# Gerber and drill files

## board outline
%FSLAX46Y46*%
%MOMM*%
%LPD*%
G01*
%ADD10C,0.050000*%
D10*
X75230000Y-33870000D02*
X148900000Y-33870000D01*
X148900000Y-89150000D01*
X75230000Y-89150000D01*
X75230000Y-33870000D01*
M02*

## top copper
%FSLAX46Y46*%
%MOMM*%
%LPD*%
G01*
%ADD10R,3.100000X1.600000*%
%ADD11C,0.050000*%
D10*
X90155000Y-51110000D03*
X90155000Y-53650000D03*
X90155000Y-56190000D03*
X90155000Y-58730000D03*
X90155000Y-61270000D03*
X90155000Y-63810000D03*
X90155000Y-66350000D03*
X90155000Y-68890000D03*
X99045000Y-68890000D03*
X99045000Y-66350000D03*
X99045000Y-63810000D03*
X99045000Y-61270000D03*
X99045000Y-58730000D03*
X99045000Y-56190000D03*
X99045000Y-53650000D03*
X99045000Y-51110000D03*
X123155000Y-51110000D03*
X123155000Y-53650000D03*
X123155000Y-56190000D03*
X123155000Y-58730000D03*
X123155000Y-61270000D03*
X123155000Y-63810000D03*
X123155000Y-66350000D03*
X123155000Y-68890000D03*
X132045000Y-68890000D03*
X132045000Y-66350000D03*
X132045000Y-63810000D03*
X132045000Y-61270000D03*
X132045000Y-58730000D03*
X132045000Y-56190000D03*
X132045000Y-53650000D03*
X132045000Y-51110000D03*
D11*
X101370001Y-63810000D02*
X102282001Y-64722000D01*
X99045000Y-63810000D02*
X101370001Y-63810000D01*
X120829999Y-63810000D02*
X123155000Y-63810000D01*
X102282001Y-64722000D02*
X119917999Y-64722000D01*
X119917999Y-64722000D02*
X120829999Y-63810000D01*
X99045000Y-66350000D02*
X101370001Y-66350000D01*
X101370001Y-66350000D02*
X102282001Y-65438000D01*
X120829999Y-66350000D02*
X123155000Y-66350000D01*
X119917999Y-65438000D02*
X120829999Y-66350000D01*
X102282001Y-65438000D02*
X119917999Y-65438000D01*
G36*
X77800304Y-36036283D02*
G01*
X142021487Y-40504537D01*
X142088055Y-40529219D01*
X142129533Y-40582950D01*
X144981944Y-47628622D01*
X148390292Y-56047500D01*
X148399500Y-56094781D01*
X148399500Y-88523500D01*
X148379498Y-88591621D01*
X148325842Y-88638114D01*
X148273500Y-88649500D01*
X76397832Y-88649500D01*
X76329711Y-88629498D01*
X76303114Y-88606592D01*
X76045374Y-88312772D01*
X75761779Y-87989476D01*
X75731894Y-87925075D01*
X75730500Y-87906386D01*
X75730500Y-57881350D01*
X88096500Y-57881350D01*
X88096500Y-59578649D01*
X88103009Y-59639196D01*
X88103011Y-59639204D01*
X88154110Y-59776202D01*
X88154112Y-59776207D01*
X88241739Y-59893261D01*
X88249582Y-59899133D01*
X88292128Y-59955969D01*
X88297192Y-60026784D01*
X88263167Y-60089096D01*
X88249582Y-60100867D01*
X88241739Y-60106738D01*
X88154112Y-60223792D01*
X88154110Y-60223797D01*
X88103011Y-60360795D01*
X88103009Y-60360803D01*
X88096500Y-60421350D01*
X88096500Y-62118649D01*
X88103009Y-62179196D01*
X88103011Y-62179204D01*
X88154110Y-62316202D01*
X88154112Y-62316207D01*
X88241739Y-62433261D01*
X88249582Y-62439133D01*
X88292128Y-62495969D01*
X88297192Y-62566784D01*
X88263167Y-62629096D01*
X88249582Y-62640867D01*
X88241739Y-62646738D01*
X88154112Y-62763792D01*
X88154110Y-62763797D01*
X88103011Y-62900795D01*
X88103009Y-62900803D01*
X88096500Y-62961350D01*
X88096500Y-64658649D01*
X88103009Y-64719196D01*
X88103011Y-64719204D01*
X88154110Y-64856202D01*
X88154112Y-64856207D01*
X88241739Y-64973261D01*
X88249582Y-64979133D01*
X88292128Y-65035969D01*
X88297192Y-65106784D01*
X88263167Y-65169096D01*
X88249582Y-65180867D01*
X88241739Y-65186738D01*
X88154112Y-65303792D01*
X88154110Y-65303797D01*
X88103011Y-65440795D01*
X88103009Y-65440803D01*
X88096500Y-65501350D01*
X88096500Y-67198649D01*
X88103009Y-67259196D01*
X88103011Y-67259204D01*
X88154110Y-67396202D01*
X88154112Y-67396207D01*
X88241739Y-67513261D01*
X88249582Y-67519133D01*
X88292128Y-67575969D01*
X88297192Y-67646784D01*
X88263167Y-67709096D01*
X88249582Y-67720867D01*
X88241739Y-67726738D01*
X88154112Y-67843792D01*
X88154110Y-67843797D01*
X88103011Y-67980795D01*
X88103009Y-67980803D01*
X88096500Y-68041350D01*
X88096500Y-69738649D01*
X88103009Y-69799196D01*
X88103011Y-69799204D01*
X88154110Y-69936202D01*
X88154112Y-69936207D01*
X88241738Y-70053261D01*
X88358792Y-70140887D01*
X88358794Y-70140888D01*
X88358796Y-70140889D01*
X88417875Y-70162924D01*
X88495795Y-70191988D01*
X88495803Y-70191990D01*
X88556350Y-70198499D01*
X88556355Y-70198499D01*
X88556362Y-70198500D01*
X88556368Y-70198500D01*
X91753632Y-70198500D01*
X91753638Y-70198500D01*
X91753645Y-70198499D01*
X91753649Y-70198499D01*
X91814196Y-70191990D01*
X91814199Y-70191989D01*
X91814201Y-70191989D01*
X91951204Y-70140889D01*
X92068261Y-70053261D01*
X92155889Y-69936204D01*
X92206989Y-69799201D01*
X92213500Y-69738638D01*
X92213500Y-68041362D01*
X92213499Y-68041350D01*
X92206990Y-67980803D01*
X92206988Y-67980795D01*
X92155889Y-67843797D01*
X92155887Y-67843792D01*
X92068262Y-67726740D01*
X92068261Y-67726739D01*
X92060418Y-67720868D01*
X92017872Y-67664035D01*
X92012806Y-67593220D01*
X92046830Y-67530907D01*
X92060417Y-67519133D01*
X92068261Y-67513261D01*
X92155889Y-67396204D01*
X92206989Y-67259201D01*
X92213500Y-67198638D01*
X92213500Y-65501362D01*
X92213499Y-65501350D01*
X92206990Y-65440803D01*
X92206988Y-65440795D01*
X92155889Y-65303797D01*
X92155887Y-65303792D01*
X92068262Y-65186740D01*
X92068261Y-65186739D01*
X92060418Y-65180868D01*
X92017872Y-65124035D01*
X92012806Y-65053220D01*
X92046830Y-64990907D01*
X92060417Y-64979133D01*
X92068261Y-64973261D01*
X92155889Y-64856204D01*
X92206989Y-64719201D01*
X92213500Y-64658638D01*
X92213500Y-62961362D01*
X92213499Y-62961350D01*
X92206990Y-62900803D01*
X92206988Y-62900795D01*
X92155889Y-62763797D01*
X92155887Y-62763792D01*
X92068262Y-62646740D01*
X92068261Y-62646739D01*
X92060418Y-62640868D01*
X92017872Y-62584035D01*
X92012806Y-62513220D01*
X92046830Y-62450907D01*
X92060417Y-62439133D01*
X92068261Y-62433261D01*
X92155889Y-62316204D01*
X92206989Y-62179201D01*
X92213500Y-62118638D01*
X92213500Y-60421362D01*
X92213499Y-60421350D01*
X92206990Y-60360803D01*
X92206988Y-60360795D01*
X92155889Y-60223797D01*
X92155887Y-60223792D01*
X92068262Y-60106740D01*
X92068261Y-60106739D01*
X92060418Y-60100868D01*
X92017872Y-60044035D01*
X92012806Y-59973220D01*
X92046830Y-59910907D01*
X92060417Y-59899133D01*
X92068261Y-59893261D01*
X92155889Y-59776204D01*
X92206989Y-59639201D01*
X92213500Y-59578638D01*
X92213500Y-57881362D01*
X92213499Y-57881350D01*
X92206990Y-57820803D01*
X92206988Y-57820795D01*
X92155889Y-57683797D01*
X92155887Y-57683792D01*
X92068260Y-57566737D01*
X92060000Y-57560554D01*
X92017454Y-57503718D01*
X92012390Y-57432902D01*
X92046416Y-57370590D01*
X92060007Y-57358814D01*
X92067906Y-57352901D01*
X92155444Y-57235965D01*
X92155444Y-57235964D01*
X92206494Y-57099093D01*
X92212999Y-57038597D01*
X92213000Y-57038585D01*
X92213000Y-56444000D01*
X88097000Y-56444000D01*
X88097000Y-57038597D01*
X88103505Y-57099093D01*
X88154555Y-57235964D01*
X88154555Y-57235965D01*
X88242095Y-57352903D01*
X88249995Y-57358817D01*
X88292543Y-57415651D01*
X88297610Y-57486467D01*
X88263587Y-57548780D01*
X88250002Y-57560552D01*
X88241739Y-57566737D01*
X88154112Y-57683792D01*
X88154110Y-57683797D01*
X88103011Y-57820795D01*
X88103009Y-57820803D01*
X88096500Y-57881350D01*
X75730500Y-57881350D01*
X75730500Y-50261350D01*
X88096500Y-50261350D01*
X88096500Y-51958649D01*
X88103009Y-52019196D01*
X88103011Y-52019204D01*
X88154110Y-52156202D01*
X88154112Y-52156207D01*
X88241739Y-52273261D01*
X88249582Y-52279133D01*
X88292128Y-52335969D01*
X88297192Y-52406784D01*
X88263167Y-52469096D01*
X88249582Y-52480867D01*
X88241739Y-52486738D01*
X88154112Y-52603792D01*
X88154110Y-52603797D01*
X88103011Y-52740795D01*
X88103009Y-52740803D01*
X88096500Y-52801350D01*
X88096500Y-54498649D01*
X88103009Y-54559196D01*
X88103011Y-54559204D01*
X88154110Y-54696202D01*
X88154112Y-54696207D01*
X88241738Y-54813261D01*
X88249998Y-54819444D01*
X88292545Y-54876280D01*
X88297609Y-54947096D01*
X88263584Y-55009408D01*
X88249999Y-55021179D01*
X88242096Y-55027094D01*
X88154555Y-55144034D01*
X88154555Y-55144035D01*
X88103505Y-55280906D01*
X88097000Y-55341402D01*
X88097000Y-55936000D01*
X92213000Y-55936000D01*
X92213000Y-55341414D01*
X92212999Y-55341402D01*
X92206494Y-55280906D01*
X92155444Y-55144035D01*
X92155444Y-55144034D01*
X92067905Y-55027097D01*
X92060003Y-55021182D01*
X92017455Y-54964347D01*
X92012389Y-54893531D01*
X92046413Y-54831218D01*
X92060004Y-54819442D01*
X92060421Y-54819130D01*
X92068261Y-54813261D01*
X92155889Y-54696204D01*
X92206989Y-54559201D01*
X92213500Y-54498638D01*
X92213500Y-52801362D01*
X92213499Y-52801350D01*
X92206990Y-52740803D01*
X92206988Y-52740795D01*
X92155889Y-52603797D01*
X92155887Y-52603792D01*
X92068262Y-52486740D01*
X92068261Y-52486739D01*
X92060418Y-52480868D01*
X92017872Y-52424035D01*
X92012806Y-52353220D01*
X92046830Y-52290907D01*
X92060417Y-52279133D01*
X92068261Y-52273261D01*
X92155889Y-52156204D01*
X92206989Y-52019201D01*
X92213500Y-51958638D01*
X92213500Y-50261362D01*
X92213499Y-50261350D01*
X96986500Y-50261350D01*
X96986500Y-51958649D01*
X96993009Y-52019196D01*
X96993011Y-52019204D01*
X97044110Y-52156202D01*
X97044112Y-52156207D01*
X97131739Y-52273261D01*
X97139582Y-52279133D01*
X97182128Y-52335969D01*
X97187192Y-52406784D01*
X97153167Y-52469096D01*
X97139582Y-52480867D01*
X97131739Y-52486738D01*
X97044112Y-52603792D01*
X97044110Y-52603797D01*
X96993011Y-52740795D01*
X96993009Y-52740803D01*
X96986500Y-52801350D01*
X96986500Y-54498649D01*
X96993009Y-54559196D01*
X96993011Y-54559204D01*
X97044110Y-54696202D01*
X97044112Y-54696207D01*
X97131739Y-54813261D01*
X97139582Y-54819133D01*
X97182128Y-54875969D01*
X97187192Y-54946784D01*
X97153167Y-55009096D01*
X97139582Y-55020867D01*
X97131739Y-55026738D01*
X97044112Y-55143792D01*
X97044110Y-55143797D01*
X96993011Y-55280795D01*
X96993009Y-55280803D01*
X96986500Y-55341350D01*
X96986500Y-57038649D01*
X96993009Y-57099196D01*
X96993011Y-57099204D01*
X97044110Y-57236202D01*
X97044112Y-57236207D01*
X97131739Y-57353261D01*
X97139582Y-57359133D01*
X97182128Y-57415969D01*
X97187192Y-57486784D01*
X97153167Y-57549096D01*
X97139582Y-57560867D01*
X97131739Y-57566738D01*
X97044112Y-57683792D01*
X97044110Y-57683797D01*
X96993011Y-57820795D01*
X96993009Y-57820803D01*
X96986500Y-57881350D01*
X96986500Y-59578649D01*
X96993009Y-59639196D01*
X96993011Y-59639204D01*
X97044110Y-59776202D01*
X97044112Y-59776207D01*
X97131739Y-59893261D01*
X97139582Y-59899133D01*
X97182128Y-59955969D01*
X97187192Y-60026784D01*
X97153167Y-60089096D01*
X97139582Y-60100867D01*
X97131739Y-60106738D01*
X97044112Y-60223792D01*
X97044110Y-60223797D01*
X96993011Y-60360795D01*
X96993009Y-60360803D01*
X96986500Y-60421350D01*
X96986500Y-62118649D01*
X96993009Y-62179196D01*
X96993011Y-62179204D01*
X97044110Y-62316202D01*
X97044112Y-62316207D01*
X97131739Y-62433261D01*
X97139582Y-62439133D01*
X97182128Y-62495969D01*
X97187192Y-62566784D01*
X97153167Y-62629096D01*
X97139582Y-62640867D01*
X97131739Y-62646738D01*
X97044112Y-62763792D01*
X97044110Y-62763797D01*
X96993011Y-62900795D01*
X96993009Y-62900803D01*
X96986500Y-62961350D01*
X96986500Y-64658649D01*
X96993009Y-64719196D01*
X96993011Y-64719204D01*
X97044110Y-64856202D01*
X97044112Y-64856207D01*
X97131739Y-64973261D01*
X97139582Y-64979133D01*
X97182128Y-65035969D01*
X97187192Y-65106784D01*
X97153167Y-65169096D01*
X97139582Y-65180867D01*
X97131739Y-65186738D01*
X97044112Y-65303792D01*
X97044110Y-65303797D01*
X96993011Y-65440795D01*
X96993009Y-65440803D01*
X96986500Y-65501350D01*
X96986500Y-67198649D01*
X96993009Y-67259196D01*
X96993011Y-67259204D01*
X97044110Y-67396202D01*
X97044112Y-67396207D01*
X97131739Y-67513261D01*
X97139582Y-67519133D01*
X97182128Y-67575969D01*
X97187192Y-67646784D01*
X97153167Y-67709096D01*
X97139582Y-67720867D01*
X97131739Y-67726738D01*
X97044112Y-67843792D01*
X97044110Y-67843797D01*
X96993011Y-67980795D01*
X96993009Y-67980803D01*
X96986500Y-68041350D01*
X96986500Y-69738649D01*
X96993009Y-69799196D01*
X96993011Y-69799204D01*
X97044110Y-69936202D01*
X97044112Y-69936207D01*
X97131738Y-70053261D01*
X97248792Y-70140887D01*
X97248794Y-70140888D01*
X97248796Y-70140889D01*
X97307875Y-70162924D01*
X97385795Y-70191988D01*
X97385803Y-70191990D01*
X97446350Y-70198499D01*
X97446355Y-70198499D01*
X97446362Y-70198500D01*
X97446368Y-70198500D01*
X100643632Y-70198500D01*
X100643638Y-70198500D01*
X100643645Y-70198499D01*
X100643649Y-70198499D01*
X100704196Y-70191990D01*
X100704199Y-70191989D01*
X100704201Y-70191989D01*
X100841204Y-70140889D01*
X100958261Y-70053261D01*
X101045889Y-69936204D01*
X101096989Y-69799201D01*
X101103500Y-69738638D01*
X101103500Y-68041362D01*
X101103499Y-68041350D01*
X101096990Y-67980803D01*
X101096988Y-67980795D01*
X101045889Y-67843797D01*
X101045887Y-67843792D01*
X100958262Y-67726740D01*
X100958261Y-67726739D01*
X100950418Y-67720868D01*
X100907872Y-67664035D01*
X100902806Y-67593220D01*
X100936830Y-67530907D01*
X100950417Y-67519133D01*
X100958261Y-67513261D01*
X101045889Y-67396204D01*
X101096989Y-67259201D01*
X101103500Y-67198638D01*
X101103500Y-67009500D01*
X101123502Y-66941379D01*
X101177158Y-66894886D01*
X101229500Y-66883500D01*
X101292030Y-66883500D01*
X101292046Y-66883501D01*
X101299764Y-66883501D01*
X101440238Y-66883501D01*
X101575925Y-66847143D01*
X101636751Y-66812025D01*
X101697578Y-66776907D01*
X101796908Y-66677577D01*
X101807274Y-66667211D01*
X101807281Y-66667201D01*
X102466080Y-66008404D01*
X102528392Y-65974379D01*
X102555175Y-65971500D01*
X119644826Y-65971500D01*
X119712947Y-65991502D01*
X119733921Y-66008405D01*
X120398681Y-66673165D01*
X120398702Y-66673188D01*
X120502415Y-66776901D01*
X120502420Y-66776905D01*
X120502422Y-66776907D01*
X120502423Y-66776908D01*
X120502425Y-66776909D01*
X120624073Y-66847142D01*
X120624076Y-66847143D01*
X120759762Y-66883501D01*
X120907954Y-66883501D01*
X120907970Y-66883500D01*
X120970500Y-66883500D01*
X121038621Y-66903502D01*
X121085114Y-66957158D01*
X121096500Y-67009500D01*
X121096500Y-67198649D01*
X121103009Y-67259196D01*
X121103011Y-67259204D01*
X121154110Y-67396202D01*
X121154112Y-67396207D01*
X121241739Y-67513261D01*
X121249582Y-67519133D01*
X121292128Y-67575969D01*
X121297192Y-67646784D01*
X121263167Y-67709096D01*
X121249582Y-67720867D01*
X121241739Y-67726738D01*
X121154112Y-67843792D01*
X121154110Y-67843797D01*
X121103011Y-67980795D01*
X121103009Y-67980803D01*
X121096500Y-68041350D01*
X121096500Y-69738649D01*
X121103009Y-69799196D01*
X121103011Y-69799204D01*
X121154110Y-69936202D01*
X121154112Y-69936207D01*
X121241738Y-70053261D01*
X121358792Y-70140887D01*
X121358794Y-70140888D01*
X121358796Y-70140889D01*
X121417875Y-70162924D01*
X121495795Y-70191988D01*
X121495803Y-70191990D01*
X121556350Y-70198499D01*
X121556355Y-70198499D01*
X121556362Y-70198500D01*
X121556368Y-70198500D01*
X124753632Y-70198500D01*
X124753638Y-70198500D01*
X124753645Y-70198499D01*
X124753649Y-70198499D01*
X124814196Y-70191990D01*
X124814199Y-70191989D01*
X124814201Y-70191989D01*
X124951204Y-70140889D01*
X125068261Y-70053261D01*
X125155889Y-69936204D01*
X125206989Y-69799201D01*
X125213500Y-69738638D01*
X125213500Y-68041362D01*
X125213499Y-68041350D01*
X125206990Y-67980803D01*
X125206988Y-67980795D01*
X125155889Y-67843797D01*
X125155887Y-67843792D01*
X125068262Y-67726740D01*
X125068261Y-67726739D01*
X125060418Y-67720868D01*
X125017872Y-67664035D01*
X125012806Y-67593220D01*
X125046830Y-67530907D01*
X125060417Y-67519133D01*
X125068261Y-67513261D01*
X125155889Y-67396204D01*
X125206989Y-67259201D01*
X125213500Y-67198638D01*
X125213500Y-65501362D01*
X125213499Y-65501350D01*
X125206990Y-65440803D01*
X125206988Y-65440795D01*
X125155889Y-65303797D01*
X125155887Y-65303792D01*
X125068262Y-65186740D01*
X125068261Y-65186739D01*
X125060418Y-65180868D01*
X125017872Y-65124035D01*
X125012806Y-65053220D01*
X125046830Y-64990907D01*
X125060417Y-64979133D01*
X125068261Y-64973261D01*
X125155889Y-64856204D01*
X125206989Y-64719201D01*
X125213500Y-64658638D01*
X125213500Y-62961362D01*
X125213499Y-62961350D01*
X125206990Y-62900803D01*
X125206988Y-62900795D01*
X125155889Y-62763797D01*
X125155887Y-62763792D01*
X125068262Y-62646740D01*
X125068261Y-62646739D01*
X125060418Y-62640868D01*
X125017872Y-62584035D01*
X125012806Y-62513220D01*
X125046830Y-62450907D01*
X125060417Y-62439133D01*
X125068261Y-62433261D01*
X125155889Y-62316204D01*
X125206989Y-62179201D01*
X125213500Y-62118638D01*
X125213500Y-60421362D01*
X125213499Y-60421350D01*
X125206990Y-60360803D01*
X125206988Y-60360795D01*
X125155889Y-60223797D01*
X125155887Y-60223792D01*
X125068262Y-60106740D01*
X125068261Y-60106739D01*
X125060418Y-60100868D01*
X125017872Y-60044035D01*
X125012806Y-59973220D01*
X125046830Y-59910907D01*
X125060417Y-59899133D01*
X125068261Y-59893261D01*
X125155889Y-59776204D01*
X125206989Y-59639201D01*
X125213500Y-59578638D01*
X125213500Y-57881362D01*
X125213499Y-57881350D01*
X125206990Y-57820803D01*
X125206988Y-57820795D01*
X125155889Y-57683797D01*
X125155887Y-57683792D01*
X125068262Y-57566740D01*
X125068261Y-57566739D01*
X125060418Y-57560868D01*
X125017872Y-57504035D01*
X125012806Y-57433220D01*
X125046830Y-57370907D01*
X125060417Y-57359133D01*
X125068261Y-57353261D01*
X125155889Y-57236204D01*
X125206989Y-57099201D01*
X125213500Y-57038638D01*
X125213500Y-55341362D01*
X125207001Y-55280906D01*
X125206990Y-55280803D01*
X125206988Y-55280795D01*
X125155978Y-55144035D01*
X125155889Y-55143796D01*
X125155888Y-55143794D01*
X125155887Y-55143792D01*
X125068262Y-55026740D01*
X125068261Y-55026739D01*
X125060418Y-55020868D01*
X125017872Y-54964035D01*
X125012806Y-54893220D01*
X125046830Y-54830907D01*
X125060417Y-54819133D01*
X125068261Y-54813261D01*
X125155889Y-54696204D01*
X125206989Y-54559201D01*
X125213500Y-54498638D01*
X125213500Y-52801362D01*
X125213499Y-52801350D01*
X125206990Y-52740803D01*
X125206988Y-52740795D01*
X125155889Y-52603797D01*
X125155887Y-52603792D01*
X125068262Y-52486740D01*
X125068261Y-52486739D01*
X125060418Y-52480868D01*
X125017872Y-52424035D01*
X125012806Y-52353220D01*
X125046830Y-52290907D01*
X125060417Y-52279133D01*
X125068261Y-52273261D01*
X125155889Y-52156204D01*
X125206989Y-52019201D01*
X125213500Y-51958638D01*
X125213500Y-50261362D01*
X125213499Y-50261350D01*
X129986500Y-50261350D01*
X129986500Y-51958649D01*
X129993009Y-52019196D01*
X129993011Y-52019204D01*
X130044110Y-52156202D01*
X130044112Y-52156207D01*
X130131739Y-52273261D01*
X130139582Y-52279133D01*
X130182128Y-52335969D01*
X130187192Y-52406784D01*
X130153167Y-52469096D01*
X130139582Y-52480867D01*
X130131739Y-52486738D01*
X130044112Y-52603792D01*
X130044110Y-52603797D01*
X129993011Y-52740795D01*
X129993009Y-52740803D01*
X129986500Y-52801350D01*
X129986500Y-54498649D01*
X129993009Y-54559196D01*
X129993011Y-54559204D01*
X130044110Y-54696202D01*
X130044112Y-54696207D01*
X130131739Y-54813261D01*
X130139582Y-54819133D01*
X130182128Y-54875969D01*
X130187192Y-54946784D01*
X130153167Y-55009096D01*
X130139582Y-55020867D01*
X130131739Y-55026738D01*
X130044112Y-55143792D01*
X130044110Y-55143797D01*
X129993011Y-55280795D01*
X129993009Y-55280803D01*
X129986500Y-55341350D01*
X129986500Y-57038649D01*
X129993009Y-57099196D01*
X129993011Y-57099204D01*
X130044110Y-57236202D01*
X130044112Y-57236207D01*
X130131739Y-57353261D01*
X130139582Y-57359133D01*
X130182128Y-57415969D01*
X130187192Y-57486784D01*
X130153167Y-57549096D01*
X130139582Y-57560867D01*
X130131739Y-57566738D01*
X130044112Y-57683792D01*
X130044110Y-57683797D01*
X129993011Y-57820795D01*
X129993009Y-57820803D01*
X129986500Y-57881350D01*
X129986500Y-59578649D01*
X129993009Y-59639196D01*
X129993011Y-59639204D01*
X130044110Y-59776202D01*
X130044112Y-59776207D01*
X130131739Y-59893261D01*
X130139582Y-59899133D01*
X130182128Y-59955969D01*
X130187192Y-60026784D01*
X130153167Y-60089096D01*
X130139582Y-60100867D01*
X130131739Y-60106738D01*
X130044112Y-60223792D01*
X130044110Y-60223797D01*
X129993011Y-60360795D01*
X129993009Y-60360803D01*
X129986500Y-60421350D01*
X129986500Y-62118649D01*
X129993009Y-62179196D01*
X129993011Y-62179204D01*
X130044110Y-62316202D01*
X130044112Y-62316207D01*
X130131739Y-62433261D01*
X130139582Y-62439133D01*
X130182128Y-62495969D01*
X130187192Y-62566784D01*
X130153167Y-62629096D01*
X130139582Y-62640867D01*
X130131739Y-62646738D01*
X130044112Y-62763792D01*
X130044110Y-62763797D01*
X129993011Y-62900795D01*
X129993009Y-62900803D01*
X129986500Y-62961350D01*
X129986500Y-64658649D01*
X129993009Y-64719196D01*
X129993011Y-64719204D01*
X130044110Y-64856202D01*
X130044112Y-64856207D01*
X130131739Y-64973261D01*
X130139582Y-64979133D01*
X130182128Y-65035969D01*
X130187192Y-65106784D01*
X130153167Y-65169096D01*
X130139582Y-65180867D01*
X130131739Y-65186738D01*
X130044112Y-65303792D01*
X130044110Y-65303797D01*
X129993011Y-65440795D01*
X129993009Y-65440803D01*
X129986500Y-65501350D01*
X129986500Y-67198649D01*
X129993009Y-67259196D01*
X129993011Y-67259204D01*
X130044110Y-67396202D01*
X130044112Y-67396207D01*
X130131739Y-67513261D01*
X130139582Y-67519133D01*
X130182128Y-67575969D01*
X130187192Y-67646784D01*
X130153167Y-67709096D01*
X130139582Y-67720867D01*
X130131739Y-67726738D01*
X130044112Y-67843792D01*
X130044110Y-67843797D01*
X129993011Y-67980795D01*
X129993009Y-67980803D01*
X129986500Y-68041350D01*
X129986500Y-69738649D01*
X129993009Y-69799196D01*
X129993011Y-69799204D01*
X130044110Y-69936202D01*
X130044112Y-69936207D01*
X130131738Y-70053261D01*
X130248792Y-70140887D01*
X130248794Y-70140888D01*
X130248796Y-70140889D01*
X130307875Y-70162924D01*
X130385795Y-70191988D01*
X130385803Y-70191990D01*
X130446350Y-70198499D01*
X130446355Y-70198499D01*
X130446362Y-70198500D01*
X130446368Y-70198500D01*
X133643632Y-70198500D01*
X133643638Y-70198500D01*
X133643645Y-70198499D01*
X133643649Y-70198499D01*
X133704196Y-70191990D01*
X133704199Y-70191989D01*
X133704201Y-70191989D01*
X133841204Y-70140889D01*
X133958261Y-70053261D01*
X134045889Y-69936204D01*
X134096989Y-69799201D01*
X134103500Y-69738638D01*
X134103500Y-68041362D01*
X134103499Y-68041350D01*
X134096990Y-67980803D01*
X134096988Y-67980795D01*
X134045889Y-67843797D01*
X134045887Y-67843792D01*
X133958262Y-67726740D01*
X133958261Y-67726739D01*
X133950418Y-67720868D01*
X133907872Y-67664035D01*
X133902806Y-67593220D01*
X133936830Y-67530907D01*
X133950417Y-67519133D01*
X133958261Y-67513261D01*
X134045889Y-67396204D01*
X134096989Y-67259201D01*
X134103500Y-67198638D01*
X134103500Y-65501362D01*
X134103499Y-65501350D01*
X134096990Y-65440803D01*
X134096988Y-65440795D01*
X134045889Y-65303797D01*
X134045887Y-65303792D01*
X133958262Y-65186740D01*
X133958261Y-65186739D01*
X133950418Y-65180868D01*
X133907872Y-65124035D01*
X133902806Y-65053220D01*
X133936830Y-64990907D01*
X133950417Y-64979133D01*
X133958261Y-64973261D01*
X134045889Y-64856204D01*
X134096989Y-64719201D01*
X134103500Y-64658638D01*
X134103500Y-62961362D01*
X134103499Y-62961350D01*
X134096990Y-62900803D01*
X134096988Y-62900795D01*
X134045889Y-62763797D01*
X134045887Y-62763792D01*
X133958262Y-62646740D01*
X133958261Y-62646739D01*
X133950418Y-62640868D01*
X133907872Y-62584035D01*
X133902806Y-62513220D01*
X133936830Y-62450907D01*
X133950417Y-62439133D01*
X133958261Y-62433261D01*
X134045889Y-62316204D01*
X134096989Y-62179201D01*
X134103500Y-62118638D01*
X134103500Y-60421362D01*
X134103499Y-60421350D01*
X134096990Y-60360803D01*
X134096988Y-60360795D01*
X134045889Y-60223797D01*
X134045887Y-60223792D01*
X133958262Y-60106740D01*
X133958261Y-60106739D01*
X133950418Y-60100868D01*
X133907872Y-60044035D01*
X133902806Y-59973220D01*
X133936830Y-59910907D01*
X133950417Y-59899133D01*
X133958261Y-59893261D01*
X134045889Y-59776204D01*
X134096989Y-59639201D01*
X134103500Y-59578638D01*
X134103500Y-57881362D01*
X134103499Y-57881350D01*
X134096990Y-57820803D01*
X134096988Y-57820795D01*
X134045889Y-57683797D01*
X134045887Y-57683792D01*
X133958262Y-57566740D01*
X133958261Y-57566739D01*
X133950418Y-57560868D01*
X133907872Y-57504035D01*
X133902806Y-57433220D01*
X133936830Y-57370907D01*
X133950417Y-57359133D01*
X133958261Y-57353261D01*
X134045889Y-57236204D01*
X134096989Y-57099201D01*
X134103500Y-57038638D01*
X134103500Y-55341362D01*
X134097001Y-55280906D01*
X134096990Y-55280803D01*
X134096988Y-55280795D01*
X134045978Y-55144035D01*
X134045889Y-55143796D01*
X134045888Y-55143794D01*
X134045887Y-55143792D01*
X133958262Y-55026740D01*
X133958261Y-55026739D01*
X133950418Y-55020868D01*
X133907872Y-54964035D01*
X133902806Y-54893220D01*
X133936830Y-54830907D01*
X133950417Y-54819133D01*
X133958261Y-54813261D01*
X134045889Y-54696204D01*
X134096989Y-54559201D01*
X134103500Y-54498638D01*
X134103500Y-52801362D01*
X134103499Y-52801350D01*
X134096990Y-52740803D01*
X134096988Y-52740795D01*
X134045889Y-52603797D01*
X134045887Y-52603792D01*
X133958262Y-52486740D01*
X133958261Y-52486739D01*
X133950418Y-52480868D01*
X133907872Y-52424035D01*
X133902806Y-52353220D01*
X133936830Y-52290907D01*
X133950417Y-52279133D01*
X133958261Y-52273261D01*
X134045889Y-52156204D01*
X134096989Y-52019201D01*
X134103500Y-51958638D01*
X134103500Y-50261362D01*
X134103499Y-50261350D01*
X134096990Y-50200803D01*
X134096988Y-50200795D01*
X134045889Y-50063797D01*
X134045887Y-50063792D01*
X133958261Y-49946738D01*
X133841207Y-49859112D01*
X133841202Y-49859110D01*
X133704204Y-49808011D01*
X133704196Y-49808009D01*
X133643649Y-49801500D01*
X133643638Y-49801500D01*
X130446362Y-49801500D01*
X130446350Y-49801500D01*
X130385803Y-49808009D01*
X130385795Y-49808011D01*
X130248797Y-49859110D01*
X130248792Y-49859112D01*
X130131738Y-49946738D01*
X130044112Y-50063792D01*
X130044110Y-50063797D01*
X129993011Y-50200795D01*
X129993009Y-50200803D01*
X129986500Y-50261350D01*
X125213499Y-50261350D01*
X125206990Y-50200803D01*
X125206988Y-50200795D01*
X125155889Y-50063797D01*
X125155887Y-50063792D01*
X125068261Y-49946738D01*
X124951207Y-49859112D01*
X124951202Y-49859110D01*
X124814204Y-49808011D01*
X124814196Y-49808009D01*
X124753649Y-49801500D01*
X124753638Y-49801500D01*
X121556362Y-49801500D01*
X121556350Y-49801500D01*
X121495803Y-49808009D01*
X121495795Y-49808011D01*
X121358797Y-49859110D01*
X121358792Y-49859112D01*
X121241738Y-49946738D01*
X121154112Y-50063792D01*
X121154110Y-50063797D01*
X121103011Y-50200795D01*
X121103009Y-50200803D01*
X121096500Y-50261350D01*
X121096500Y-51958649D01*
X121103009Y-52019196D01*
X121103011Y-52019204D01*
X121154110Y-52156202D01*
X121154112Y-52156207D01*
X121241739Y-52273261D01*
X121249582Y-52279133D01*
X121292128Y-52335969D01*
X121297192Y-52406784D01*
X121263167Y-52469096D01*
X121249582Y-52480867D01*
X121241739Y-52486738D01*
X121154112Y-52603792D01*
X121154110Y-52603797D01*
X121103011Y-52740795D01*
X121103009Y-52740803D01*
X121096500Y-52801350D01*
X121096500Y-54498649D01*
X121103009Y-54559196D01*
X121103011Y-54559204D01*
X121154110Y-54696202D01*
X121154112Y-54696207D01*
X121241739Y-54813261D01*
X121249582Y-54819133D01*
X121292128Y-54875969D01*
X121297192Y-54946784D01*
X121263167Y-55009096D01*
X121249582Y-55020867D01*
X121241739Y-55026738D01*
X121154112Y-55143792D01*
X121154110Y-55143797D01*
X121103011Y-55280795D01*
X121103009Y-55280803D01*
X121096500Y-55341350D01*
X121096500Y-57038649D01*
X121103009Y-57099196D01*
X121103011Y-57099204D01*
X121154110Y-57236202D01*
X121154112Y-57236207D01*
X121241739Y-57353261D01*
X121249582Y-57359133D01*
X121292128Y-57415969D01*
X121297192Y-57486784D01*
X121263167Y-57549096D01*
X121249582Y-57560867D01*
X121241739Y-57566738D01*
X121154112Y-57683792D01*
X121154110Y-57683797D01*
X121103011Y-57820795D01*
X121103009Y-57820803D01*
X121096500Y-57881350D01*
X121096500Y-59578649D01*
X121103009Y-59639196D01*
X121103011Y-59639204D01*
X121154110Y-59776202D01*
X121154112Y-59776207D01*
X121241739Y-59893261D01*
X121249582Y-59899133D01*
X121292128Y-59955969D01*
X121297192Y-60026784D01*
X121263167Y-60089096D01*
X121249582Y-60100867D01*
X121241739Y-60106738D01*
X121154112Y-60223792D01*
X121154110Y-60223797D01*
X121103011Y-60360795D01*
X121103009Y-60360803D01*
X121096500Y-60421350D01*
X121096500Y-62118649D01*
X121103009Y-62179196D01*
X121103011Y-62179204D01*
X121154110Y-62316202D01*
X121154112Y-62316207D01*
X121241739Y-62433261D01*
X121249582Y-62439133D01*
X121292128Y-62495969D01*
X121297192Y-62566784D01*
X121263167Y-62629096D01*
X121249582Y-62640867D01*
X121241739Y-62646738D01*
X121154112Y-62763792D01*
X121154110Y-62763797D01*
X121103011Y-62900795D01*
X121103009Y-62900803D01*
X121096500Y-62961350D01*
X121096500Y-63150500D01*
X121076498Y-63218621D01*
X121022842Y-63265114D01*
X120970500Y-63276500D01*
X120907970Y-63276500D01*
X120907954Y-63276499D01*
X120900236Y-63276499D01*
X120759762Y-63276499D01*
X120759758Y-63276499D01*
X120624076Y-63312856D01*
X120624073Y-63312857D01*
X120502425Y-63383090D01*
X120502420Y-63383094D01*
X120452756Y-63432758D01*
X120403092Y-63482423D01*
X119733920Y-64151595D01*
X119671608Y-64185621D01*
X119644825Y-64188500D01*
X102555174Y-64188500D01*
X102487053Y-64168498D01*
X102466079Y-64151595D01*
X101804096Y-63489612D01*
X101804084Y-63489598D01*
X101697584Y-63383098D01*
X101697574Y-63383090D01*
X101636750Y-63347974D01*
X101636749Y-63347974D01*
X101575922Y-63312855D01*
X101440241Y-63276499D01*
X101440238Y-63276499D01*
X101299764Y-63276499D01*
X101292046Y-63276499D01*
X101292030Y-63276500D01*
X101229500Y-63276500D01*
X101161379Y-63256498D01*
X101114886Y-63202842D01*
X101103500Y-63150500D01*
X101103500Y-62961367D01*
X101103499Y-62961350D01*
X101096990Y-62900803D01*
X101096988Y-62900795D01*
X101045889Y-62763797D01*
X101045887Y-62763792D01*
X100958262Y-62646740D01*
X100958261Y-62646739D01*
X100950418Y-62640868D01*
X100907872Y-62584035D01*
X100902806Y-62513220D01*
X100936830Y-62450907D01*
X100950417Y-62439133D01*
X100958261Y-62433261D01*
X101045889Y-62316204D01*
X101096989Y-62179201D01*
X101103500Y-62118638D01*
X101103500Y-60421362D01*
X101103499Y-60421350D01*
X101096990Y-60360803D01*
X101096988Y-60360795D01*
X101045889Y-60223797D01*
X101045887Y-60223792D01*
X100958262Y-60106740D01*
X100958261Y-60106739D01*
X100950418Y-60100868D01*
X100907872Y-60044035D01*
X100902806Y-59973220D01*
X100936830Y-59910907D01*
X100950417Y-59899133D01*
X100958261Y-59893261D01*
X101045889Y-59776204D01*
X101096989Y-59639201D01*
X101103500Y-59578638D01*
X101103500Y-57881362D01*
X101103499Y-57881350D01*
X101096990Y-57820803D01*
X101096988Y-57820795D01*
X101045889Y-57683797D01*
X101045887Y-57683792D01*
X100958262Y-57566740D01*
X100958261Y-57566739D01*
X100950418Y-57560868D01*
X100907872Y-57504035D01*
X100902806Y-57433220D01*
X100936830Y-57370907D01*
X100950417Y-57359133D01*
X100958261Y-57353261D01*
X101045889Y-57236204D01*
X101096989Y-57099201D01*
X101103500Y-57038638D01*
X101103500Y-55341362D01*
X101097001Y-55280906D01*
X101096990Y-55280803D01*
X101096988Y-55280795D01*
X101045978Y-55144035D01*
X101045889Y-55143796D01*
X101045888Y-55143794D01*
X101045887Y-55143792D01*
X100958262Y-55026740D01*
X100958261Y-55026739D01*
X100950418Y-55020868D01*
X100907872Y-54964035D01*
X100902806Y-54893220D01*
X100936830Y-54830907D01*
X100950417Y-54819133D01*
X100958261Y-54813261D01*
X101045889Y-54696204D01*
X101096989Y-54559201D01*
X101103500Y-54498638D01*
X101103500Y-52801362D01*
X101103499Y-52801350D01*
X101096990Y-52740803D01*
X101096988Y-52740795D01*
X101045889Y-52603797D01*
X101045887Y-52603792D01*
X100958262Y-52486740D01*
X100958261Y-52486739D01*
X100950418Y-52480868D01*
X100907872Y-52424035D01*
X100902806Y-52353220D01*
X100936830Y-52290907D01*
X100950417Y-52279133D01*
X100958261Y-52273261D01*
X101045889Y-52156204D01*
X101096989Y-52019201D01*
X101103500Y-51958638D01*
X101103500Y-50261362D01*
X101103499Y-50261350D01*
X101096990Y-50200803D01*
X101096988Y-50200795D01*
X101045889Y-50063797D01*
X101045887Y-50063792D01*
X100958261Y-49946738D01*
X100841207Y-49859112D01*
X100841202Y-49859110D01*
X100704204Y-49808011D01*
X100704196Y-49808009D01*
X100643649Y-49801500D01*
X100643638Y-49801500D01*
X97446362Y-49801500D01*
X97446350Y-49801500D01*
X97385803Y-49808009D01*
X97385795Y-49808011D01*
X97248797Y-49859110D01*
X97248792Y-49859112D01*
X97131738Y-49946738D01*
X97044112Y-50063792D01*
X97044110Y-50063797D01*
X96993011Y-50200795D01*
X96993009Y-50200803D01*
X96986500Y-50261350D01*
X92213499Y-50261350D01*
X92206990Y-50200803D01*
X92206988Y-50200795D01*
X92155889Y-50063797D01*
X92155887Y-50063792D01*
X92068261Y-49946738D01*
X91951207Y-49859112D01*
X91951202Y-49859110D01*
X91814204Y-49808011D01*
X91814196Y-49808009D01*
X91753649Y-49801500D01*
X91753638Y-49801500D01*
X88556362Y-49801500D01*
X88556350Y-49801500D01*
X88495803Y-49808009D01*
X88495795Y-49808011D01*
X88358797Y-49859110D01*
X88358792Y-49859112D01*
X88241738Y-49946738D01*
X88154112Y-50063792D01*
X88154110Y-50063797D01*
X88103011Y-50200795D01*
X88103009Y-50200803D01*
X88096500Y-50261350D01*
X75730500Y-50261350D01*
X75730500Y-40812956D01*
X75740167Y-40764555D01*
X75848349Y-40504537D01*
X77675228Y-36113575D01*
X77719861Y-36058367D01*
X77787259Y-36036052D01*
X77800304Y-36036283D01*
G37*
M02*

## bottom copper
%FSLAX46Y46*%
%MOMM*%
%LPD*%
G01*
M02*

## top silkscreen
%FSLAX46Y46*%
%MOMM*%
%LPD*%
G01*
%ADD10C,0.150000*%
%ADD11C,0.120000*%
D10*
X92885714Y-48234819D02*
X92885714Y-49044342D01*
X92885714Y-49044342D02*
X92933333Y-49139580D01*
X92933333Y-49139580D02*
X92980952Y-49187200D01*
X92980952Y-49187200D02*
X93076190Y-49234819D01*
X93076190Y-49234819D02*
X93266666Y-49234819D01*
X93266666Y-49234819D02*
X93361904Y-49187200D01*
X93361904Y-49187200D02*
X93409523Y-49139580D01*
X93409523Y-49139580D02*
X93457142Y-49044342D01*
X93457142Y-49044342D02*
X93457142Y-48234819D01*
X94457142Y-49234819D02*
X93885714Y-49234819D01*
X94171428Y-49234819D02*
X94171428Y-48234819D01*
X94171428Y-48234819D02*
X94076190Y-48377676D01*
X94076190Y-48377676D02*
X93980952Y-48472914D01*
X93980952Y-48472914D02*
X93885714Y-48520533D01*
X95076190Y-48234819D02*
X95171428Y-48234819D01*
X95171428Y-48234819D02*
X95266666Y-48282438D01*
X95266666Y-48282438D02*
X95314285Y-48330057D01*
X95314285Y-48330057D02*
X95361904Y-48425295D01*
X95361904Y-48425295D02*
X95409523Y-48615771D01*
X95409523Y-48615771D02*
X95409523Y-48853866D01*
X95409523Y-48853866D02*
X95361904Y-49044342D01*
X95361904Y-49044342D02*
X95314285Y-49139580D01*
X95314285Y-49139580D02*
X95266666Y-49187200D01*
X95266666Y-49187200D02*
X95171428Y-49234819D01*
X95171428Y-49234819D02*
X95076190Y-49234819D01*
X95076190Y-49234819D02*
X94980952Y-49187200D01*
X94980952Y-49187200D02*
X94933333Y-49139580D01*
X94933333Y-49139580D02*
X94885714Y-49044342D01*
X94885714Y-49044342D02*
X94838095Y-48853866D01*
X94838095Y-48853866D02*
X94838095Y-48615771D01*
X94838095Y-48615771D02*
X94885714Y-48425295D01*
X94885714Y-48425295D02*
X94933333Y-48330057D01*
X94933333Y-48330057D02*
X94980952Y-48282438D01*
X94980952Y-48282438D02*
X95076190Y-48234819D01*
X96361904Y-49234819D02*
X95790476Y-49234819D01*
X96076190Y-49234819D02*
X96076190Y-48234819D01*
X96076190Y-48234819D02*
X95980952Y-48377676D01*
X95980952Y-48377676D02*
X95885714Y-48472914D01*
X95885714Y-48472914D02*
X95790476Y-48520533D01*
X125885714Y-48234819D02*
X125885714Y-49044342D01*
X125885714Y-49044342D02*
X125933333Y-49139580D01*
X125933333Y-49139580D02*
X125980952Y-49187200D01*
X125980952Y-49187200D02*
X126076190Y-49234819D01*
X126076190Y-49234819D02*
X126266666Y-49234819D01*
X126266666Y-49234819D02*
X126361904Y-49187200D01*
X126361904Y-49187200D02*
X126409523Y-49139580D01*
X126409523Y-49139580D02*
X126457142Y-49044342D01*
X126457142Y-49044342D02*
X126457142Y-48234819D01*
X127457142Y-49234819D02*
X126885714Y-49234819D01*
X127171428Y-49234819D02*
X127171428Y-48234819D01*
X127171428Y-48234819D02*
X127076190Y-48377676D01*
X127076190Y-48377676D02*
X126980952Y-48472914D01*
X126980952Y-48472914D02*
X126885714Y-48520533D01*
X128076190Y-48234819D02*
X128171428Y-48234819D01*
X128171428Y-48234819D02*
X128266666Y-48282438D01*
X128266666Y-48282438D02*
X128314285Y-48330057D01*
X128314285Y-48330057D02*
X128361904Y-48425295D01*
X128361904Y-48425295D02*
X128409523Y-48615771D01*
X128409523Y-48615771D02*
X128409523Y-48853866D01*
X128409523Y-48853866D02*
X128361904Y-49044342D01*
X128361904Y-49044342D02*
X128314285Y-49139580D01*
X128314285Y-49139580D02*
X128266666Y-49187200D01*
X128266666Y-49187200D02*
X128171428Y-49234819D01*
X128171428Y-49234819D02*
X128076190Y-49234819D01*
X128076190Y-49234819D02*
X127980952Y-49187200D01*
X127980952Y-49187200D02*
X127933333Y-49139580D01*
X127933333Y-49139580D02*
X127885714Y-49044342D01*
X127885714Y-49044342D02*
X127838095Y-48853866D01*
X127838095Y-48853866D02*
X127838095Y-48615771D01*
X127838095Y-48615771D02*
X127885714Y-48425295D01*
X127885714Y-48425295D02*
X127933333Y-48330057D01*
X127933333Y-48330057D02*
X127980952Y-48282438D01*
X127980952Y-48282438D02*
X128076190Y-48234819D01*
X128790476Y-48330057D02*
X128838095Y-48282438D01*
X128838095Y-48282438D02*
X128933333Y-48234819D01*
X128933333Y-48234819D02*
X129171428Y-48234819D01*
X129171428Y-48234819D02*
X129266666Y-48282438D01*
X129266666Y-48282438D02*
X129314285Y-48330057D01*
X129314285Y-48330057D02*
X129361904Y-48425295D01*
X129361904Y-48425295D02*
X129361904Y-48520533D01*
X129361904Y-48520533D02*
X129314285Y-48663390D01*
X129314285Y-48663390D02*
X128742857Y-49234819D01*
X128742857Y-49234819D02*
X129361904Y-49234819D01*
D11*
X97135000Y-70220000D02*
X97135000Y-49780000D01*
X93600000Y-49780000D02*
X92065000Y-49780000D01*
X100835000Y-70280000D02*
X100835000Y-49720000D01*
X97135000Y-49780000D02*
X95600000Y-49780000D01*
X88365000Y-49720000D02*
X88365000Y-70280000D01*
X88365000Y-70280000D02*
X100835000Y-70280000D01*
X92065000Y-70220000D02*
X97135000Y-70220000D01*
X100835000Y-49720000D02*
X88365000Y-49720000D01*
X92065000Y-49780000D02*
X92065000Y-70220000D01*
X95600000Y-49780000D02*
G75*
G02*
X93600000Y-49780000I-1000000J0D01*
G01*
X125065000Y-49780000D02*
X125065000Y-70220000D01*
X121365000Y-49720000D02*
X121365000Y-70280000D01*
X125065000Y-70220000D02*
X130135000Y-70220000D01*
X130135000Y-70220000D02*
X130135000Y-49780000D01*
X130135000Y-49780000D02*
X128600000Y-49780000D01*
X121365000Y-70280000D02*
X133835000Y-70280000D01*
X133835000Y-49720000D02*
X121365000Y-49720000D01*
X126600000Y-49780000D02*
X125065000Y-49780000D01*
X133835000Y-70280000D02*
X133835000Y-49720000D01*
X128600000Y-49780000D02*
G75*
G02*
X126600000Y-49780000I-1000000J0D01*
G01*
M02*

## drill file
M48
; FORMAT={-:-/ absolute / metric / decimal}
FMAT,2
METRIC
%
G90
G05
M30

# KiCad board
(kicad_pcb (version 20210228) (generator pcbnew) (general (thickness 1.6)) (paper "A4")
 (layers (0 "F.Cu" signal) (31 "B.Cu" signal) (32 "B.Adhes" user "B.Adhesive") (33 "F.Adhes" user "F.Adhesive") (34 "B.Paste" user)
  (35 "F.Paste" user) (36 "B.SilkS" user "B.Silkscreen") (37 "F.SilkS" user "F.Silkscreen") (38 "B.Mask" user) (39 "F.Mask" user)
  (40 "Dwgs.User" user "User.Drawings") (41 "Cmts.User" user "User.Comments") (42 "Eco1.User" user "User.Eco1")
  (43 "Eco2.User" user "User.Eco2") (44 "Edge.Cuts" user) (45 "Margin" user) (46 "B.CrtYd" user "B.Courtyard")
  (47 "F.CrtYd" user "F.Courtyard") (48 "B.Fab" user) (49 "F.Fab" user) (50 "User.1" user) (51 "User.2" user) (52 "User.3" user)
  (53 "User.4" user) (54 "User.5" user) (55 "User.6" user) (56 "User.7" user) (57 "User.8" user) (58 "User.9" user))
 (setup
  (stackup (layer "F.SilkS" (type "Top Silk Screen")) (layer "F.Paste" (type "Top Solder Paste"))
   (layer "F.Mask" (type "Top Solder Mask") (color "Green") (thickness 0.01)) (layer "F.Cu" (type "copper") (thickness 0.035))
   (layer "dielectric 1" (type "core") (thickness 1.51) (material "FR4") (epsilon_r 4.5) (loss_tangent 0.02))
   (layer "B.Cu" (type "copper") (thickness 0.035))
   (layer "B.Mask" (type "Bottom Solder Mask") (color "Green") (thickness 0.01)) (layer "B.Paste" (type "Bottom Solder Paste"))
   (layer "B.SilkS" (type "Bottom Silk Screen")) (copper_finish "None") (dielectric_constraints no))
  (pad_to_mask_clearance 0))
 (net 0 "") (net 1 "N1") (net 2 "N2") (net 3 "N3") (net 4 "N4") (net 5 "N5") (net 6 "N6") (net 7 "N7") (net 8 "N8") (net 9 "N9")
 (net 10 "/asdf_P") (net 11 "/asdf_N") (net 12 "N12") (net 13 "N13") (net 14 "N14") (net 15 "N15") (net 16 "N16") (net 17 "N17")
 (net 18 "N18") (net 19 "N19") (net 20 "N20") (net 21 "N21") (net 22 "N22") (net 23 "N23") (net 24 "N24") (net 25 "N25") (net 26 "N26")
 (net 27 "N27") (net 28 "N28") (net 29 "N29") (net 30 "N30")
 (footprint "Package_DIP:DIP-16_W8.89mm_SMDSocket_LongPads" (layer "F.Cu") (at 94.6 60)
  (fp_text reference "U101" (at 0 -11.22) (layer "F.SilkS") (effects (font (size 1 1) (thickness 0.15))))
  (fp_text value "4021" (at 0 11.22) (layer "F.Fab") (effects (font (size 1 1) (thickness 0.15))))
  (fp_line (start 2.535 10.22) (end 2.535 -10.22) (layer "F.SilkS") (width 0.12))
  (fp_line (start -1 -10.22) (end -2.535 -10.22) (layer "F.SilkS") (width 0.12))
  (fp_line (start 6.235 10.28) (end 6.235 -10.28) (layer "F.SilkS") (width 0.12))
  (fp_line (start 2.535 -10.22) (end 1 -10.22) (layer "F.SilkS") (width 0.12))
  (fp_line (start -6.235 -10.28) (end -6.235 10.28) (layer "F.SilkS") (width 0.12))
  (fp_line (start -6.235 10.28) (end 6.235 10.28) (layer "F.SilkS") (width 0.12))
  (fp_line (start -2.535 10.22) (end 2.535 10.22) (layer "F.SilkS") (width 0.12))
  (fp_line (start 6.235 -10.28) (end -6.235 -10.28) (layer "F.SilkS") (width 0.12))
  (fp_line (start -2.535 -10.22) (end -2.535 10.22) (layer "F.SilkS") (width 0.12))
  (fp_arc (start 0 -10.22) (end -1 -10.22) (angle -180) (layer "F.SilkS") (width 0.12))
  (pad "1" smd rect (at -4.445 -8.89) (locked) (size 3.1 1.6) (layers "F.Cu" "F.Paste" "F.Mask") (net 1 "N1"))
  (pad "2" smd rect (at -4.445 -6.35) (locked) (size 3.1 1.6) (layers "F.Cu" "F.Paste" "F.Mask") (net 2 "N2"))
  (pad "3" smd rect (at -4.445 -3.81) (locked) (size 3.1 1.6) (layers "F.Cu" "F.Paste" "F.Mask") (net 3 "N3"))
  (pad "4" smd rect (at -4.445 -1.27) (locked) (size 3.1 1.6) (layers "F.Cu" "F.Paste" "F.Mask") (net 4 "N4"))
  (pad "5" smd rect (at -4.445 1.27) (locked) (size 3.1 1.6) (layers "F.Cu" "F.Paste" "F.Mask") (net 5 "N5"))
  (pad "6" smd rect (at -4.445 3.81) (locked) (size 3.1 1.6) (layers "F.Cu" "F.Paste" "F.Mask") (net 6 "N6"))
  (pad "7" smd rect (at -4.445 6.35) (locked) (size 3.1 1.6) (layers "F.Cu" "F.Paste" "F.Mask") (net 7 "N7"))
  (pad "8" smd rect (at -4.445 8.89) (locked) (size 3.1 1.6) (layers "F.Cu" "F.Paste" "F.Mask") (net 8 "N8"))
  (pad "9" smd rect (at 4.445 8.89) (locked) (size 3.1 1.6) (layers "F.Cu" "F.Paste" "F.Mask") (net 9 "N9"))
  (pad "10" smd rect (at 4.445 6.35) (locked) (size 3.1 1.6) (layers "F.Cu" "F.Paste" "F.Mask") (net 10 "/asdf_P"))
  (pad "11" smd rect (at 4.445 3.81) (locked) (size 3.1 1.6) (layers "F.Cu" "F.Paste" "F.Mask") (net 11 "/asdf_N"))
  (pad "12" smd rect (at 4.445 1.27) (locked) (size 3.1 1.6) (layers "F.Cu" "F.Paste" "F.Mask") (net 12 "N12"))
  (pad "13" smd rect (at 4.445 -1.27) (locked) (size 3.1 1.6) (layers "F.Cu" "F.Paste" "F.Mask") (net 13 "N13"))
  (pad "14" smd rect (at 4.445 -3.81) (locked) (size 3.1 1.6) (layers "F.Cu" "F.Paste" "F.Mask") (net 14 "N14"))
  (pad "15" smd rect (at 4.445 -6.35) (locked) (size 3.1 1.6) (layers "F.Cu" "F.Paste" "F.Mask") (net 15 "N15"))
  (pad "16" smd rect (at 4.445 -8.89) (locked) (size 3.1 1.6) (layers "F.Cu" "F.Paste" "F.Mask") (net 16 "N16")))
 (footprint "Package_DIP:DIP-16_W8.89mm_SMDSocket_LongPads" (layer "F.Cu") (at 127.6 60)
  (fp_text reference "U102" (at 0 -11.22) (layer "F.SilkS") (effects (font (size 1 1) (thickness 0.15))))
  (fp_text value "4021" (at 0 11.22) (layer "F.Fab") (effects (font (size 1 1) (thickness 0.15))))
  (fp_line (start -2.535 -10.22) (end -2.535 10.22) (layer "F.SilkS") (width 0.12))
  (fp_line (start -6.235 -10.28) (end -6.235 10.28) (layer "F.SilkS") (width 0.12))
  (fp_line (start -2.535 10.22) (end 2.535 10.22) (layer "F.SilkS") (width 0.12))
  (fp_line (start 2.535 10.22) (end 2.535 -10.22) (layer "F.SilkS") (width 0.12))
  (fp_line (start 2.535 -10.22) (end 1 -10.22) (layer "F.SilkS") (width 0.12))
  (fp_line (start -6.235 10.28) (end 6.235 10.28) (layer "F.SilkS") (width 0.12))
  (fp_line (start 6.235 -10.28) (end -6.235 -10.28) (layer "F.SilkS") (width 0.12))
  (fp_line (start -1 -10.22) (end -2.535 -10.22) (layer "F.SilkS") (width 0.12))
  (fp_line (start 6.235 10.28) (end 6.235 -10.28) (layer "F.SilkS") (width 0.12))
  (fp_arc (start 0 -10.22) (end -1 -10.22) (angle -180) (layer "F.SilkS") (width 0.12))
  (pad "1" smd rect (at -4.445 -8.89) (locked) (size 3.1 1.6) (layers "F.Cu" "F.Paste" "F.Mask") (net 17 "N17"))
  (pad "2" smd rect (at -4.445 -6.35) (locked) (size 3.1 1.6) (layers "F.Cu" "F.Paste" "F.Mask") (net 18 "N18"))
  (pad "3" smd rect (at -4.445 -3.81) (locked) (size 3.1 1.6) (layers "F.Cu" "F.Paste" "F.Mask") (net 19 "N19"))
  (pad "4" smd rect (at -4.445 -1.27) (locked) (size 3.1 1.6) (layers "F.Cu" "F.Paste" "F.Mask") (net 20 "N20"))
  (pad "5" smd rect (at -4.445 1.27) (locked) (size 3.1 1.6) (layers "F.Cu" "F.Paste" "F.Mask") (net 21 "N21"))
  (pad "6" smd rect (at -4.445 3.81) (locked) (size 3.1 1.6) (layers "F.Cu" "F.Paste" "F.Mask") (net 11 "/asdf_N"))
  (pad "7" smd rect (at -4.445 6.35) (locked) (size 3.1 1.6) (layers "F.Cu" "F.Paste" "F.Mask") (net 10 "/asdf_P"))
  (pad "8" smd rect (at -4.445 8.89) (locked) (size 3.1 1.6) (layers "F.Cu" "F.Paste" "F.Mask") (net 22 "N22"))
  (pad "9" smd rect (at 4.445 8.89) (locked) (size 3.1 1.6) (layers "F.Cu" "F.Paste" "F.Mask") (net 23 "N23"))
  (pad "10" smd rect (at 4.445 6.35) (locked) (size 3.1 1.6) (layers "F.Cu" "F.Paste" "F.Mask") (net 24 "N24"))
  (pad "11" smd rect (at 4.445 3.81) (locked) (size 3.1 1.6) (layers "F.Cu" "F.Paste" "F.Mask") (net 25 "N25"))
  (pad "12" smd rect (at 4.445 1.27) (locked) (size 3.1 1.6) (layers "F.Cu" "F.Paste" "F.Mask") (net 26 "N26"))
  (pad "13" smd rect (at 4.445 -1.27) (locked) (size 3.1 1.6) (layers "F.Cu" "F.Paste" "F.Mask") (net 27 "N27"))
  (pad "14" smd rect (at 4.445 -3.81) (locked) (size 3.1 1.6) (layers "F.Cu" "F.Paste" "F.Mask") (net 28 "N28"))
  (pad "15" smd rect (at 4.445 -6.35) (locked) (size 3.1 1.6) (layers "F.Cu" "F.Paste" "F.Mask") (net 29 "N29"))
  (pad "16" smd rect (at 4.445 -8.89) (locked) (size 3.1 1.6) (layers "F.Cu" "F.Paste" "F.Mask") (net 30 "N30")))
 (gr_rect (start 75.23 33.87) (end 148.9 89.15) (layer "Edge.Cuts") (width 0.05) (fill none))
 (segment (start 101.370001 63.81) (end 102.282001 64.722) (width 0.05) (layer "F.Cu") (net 11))
 (segment (start 99.045 63.81) (end 101.370001 63.81) (width 0.05) (layer "F.Cu") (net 11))
 (segment (start 120.829999 63.81) (end 123.155 63.81) (width 0.05) (layer "F.Cu") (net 11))
 (segment (start 102.282001 64.722) (end 119.917999 64.722) (width 0.05) (layer "F.Cu") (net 11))
 (segment (start 119.917999 64.722) (end 120.829999 63.81) (width 0.05) (layer "F.Cu") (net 11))
 (segment (start 99.045 66.35) (end 101.370001 66.35) (width 0.05) (layer "F.Cu") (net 10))
 (segment (start 101.370001 66.35) (end 102.282001 65.438) (width 0.05) (layer "F.Cu") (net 10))
 (segment (start 120.829999 66.35) (end 123.155 66.35) (width 0.05) (layer "F.Cu") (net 10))
 (segment (start 119.917999 65.438) (end 120.829999 66.35) (width 0.05) (layer "F.Cu") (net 10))
 (segment (start 102.282001 65.438) (end 119.917999 65.438) (width 0.05) (layer "F.Cu") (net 10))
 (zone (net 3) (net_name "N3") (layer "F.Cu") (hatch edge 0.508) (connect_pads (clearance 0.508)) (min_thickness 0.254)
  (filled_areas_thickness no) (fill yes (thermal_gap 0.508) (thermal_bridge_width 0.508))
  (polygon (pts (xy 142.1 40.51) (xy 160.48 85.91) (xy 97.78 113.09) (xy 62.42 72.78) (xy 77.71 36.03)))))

